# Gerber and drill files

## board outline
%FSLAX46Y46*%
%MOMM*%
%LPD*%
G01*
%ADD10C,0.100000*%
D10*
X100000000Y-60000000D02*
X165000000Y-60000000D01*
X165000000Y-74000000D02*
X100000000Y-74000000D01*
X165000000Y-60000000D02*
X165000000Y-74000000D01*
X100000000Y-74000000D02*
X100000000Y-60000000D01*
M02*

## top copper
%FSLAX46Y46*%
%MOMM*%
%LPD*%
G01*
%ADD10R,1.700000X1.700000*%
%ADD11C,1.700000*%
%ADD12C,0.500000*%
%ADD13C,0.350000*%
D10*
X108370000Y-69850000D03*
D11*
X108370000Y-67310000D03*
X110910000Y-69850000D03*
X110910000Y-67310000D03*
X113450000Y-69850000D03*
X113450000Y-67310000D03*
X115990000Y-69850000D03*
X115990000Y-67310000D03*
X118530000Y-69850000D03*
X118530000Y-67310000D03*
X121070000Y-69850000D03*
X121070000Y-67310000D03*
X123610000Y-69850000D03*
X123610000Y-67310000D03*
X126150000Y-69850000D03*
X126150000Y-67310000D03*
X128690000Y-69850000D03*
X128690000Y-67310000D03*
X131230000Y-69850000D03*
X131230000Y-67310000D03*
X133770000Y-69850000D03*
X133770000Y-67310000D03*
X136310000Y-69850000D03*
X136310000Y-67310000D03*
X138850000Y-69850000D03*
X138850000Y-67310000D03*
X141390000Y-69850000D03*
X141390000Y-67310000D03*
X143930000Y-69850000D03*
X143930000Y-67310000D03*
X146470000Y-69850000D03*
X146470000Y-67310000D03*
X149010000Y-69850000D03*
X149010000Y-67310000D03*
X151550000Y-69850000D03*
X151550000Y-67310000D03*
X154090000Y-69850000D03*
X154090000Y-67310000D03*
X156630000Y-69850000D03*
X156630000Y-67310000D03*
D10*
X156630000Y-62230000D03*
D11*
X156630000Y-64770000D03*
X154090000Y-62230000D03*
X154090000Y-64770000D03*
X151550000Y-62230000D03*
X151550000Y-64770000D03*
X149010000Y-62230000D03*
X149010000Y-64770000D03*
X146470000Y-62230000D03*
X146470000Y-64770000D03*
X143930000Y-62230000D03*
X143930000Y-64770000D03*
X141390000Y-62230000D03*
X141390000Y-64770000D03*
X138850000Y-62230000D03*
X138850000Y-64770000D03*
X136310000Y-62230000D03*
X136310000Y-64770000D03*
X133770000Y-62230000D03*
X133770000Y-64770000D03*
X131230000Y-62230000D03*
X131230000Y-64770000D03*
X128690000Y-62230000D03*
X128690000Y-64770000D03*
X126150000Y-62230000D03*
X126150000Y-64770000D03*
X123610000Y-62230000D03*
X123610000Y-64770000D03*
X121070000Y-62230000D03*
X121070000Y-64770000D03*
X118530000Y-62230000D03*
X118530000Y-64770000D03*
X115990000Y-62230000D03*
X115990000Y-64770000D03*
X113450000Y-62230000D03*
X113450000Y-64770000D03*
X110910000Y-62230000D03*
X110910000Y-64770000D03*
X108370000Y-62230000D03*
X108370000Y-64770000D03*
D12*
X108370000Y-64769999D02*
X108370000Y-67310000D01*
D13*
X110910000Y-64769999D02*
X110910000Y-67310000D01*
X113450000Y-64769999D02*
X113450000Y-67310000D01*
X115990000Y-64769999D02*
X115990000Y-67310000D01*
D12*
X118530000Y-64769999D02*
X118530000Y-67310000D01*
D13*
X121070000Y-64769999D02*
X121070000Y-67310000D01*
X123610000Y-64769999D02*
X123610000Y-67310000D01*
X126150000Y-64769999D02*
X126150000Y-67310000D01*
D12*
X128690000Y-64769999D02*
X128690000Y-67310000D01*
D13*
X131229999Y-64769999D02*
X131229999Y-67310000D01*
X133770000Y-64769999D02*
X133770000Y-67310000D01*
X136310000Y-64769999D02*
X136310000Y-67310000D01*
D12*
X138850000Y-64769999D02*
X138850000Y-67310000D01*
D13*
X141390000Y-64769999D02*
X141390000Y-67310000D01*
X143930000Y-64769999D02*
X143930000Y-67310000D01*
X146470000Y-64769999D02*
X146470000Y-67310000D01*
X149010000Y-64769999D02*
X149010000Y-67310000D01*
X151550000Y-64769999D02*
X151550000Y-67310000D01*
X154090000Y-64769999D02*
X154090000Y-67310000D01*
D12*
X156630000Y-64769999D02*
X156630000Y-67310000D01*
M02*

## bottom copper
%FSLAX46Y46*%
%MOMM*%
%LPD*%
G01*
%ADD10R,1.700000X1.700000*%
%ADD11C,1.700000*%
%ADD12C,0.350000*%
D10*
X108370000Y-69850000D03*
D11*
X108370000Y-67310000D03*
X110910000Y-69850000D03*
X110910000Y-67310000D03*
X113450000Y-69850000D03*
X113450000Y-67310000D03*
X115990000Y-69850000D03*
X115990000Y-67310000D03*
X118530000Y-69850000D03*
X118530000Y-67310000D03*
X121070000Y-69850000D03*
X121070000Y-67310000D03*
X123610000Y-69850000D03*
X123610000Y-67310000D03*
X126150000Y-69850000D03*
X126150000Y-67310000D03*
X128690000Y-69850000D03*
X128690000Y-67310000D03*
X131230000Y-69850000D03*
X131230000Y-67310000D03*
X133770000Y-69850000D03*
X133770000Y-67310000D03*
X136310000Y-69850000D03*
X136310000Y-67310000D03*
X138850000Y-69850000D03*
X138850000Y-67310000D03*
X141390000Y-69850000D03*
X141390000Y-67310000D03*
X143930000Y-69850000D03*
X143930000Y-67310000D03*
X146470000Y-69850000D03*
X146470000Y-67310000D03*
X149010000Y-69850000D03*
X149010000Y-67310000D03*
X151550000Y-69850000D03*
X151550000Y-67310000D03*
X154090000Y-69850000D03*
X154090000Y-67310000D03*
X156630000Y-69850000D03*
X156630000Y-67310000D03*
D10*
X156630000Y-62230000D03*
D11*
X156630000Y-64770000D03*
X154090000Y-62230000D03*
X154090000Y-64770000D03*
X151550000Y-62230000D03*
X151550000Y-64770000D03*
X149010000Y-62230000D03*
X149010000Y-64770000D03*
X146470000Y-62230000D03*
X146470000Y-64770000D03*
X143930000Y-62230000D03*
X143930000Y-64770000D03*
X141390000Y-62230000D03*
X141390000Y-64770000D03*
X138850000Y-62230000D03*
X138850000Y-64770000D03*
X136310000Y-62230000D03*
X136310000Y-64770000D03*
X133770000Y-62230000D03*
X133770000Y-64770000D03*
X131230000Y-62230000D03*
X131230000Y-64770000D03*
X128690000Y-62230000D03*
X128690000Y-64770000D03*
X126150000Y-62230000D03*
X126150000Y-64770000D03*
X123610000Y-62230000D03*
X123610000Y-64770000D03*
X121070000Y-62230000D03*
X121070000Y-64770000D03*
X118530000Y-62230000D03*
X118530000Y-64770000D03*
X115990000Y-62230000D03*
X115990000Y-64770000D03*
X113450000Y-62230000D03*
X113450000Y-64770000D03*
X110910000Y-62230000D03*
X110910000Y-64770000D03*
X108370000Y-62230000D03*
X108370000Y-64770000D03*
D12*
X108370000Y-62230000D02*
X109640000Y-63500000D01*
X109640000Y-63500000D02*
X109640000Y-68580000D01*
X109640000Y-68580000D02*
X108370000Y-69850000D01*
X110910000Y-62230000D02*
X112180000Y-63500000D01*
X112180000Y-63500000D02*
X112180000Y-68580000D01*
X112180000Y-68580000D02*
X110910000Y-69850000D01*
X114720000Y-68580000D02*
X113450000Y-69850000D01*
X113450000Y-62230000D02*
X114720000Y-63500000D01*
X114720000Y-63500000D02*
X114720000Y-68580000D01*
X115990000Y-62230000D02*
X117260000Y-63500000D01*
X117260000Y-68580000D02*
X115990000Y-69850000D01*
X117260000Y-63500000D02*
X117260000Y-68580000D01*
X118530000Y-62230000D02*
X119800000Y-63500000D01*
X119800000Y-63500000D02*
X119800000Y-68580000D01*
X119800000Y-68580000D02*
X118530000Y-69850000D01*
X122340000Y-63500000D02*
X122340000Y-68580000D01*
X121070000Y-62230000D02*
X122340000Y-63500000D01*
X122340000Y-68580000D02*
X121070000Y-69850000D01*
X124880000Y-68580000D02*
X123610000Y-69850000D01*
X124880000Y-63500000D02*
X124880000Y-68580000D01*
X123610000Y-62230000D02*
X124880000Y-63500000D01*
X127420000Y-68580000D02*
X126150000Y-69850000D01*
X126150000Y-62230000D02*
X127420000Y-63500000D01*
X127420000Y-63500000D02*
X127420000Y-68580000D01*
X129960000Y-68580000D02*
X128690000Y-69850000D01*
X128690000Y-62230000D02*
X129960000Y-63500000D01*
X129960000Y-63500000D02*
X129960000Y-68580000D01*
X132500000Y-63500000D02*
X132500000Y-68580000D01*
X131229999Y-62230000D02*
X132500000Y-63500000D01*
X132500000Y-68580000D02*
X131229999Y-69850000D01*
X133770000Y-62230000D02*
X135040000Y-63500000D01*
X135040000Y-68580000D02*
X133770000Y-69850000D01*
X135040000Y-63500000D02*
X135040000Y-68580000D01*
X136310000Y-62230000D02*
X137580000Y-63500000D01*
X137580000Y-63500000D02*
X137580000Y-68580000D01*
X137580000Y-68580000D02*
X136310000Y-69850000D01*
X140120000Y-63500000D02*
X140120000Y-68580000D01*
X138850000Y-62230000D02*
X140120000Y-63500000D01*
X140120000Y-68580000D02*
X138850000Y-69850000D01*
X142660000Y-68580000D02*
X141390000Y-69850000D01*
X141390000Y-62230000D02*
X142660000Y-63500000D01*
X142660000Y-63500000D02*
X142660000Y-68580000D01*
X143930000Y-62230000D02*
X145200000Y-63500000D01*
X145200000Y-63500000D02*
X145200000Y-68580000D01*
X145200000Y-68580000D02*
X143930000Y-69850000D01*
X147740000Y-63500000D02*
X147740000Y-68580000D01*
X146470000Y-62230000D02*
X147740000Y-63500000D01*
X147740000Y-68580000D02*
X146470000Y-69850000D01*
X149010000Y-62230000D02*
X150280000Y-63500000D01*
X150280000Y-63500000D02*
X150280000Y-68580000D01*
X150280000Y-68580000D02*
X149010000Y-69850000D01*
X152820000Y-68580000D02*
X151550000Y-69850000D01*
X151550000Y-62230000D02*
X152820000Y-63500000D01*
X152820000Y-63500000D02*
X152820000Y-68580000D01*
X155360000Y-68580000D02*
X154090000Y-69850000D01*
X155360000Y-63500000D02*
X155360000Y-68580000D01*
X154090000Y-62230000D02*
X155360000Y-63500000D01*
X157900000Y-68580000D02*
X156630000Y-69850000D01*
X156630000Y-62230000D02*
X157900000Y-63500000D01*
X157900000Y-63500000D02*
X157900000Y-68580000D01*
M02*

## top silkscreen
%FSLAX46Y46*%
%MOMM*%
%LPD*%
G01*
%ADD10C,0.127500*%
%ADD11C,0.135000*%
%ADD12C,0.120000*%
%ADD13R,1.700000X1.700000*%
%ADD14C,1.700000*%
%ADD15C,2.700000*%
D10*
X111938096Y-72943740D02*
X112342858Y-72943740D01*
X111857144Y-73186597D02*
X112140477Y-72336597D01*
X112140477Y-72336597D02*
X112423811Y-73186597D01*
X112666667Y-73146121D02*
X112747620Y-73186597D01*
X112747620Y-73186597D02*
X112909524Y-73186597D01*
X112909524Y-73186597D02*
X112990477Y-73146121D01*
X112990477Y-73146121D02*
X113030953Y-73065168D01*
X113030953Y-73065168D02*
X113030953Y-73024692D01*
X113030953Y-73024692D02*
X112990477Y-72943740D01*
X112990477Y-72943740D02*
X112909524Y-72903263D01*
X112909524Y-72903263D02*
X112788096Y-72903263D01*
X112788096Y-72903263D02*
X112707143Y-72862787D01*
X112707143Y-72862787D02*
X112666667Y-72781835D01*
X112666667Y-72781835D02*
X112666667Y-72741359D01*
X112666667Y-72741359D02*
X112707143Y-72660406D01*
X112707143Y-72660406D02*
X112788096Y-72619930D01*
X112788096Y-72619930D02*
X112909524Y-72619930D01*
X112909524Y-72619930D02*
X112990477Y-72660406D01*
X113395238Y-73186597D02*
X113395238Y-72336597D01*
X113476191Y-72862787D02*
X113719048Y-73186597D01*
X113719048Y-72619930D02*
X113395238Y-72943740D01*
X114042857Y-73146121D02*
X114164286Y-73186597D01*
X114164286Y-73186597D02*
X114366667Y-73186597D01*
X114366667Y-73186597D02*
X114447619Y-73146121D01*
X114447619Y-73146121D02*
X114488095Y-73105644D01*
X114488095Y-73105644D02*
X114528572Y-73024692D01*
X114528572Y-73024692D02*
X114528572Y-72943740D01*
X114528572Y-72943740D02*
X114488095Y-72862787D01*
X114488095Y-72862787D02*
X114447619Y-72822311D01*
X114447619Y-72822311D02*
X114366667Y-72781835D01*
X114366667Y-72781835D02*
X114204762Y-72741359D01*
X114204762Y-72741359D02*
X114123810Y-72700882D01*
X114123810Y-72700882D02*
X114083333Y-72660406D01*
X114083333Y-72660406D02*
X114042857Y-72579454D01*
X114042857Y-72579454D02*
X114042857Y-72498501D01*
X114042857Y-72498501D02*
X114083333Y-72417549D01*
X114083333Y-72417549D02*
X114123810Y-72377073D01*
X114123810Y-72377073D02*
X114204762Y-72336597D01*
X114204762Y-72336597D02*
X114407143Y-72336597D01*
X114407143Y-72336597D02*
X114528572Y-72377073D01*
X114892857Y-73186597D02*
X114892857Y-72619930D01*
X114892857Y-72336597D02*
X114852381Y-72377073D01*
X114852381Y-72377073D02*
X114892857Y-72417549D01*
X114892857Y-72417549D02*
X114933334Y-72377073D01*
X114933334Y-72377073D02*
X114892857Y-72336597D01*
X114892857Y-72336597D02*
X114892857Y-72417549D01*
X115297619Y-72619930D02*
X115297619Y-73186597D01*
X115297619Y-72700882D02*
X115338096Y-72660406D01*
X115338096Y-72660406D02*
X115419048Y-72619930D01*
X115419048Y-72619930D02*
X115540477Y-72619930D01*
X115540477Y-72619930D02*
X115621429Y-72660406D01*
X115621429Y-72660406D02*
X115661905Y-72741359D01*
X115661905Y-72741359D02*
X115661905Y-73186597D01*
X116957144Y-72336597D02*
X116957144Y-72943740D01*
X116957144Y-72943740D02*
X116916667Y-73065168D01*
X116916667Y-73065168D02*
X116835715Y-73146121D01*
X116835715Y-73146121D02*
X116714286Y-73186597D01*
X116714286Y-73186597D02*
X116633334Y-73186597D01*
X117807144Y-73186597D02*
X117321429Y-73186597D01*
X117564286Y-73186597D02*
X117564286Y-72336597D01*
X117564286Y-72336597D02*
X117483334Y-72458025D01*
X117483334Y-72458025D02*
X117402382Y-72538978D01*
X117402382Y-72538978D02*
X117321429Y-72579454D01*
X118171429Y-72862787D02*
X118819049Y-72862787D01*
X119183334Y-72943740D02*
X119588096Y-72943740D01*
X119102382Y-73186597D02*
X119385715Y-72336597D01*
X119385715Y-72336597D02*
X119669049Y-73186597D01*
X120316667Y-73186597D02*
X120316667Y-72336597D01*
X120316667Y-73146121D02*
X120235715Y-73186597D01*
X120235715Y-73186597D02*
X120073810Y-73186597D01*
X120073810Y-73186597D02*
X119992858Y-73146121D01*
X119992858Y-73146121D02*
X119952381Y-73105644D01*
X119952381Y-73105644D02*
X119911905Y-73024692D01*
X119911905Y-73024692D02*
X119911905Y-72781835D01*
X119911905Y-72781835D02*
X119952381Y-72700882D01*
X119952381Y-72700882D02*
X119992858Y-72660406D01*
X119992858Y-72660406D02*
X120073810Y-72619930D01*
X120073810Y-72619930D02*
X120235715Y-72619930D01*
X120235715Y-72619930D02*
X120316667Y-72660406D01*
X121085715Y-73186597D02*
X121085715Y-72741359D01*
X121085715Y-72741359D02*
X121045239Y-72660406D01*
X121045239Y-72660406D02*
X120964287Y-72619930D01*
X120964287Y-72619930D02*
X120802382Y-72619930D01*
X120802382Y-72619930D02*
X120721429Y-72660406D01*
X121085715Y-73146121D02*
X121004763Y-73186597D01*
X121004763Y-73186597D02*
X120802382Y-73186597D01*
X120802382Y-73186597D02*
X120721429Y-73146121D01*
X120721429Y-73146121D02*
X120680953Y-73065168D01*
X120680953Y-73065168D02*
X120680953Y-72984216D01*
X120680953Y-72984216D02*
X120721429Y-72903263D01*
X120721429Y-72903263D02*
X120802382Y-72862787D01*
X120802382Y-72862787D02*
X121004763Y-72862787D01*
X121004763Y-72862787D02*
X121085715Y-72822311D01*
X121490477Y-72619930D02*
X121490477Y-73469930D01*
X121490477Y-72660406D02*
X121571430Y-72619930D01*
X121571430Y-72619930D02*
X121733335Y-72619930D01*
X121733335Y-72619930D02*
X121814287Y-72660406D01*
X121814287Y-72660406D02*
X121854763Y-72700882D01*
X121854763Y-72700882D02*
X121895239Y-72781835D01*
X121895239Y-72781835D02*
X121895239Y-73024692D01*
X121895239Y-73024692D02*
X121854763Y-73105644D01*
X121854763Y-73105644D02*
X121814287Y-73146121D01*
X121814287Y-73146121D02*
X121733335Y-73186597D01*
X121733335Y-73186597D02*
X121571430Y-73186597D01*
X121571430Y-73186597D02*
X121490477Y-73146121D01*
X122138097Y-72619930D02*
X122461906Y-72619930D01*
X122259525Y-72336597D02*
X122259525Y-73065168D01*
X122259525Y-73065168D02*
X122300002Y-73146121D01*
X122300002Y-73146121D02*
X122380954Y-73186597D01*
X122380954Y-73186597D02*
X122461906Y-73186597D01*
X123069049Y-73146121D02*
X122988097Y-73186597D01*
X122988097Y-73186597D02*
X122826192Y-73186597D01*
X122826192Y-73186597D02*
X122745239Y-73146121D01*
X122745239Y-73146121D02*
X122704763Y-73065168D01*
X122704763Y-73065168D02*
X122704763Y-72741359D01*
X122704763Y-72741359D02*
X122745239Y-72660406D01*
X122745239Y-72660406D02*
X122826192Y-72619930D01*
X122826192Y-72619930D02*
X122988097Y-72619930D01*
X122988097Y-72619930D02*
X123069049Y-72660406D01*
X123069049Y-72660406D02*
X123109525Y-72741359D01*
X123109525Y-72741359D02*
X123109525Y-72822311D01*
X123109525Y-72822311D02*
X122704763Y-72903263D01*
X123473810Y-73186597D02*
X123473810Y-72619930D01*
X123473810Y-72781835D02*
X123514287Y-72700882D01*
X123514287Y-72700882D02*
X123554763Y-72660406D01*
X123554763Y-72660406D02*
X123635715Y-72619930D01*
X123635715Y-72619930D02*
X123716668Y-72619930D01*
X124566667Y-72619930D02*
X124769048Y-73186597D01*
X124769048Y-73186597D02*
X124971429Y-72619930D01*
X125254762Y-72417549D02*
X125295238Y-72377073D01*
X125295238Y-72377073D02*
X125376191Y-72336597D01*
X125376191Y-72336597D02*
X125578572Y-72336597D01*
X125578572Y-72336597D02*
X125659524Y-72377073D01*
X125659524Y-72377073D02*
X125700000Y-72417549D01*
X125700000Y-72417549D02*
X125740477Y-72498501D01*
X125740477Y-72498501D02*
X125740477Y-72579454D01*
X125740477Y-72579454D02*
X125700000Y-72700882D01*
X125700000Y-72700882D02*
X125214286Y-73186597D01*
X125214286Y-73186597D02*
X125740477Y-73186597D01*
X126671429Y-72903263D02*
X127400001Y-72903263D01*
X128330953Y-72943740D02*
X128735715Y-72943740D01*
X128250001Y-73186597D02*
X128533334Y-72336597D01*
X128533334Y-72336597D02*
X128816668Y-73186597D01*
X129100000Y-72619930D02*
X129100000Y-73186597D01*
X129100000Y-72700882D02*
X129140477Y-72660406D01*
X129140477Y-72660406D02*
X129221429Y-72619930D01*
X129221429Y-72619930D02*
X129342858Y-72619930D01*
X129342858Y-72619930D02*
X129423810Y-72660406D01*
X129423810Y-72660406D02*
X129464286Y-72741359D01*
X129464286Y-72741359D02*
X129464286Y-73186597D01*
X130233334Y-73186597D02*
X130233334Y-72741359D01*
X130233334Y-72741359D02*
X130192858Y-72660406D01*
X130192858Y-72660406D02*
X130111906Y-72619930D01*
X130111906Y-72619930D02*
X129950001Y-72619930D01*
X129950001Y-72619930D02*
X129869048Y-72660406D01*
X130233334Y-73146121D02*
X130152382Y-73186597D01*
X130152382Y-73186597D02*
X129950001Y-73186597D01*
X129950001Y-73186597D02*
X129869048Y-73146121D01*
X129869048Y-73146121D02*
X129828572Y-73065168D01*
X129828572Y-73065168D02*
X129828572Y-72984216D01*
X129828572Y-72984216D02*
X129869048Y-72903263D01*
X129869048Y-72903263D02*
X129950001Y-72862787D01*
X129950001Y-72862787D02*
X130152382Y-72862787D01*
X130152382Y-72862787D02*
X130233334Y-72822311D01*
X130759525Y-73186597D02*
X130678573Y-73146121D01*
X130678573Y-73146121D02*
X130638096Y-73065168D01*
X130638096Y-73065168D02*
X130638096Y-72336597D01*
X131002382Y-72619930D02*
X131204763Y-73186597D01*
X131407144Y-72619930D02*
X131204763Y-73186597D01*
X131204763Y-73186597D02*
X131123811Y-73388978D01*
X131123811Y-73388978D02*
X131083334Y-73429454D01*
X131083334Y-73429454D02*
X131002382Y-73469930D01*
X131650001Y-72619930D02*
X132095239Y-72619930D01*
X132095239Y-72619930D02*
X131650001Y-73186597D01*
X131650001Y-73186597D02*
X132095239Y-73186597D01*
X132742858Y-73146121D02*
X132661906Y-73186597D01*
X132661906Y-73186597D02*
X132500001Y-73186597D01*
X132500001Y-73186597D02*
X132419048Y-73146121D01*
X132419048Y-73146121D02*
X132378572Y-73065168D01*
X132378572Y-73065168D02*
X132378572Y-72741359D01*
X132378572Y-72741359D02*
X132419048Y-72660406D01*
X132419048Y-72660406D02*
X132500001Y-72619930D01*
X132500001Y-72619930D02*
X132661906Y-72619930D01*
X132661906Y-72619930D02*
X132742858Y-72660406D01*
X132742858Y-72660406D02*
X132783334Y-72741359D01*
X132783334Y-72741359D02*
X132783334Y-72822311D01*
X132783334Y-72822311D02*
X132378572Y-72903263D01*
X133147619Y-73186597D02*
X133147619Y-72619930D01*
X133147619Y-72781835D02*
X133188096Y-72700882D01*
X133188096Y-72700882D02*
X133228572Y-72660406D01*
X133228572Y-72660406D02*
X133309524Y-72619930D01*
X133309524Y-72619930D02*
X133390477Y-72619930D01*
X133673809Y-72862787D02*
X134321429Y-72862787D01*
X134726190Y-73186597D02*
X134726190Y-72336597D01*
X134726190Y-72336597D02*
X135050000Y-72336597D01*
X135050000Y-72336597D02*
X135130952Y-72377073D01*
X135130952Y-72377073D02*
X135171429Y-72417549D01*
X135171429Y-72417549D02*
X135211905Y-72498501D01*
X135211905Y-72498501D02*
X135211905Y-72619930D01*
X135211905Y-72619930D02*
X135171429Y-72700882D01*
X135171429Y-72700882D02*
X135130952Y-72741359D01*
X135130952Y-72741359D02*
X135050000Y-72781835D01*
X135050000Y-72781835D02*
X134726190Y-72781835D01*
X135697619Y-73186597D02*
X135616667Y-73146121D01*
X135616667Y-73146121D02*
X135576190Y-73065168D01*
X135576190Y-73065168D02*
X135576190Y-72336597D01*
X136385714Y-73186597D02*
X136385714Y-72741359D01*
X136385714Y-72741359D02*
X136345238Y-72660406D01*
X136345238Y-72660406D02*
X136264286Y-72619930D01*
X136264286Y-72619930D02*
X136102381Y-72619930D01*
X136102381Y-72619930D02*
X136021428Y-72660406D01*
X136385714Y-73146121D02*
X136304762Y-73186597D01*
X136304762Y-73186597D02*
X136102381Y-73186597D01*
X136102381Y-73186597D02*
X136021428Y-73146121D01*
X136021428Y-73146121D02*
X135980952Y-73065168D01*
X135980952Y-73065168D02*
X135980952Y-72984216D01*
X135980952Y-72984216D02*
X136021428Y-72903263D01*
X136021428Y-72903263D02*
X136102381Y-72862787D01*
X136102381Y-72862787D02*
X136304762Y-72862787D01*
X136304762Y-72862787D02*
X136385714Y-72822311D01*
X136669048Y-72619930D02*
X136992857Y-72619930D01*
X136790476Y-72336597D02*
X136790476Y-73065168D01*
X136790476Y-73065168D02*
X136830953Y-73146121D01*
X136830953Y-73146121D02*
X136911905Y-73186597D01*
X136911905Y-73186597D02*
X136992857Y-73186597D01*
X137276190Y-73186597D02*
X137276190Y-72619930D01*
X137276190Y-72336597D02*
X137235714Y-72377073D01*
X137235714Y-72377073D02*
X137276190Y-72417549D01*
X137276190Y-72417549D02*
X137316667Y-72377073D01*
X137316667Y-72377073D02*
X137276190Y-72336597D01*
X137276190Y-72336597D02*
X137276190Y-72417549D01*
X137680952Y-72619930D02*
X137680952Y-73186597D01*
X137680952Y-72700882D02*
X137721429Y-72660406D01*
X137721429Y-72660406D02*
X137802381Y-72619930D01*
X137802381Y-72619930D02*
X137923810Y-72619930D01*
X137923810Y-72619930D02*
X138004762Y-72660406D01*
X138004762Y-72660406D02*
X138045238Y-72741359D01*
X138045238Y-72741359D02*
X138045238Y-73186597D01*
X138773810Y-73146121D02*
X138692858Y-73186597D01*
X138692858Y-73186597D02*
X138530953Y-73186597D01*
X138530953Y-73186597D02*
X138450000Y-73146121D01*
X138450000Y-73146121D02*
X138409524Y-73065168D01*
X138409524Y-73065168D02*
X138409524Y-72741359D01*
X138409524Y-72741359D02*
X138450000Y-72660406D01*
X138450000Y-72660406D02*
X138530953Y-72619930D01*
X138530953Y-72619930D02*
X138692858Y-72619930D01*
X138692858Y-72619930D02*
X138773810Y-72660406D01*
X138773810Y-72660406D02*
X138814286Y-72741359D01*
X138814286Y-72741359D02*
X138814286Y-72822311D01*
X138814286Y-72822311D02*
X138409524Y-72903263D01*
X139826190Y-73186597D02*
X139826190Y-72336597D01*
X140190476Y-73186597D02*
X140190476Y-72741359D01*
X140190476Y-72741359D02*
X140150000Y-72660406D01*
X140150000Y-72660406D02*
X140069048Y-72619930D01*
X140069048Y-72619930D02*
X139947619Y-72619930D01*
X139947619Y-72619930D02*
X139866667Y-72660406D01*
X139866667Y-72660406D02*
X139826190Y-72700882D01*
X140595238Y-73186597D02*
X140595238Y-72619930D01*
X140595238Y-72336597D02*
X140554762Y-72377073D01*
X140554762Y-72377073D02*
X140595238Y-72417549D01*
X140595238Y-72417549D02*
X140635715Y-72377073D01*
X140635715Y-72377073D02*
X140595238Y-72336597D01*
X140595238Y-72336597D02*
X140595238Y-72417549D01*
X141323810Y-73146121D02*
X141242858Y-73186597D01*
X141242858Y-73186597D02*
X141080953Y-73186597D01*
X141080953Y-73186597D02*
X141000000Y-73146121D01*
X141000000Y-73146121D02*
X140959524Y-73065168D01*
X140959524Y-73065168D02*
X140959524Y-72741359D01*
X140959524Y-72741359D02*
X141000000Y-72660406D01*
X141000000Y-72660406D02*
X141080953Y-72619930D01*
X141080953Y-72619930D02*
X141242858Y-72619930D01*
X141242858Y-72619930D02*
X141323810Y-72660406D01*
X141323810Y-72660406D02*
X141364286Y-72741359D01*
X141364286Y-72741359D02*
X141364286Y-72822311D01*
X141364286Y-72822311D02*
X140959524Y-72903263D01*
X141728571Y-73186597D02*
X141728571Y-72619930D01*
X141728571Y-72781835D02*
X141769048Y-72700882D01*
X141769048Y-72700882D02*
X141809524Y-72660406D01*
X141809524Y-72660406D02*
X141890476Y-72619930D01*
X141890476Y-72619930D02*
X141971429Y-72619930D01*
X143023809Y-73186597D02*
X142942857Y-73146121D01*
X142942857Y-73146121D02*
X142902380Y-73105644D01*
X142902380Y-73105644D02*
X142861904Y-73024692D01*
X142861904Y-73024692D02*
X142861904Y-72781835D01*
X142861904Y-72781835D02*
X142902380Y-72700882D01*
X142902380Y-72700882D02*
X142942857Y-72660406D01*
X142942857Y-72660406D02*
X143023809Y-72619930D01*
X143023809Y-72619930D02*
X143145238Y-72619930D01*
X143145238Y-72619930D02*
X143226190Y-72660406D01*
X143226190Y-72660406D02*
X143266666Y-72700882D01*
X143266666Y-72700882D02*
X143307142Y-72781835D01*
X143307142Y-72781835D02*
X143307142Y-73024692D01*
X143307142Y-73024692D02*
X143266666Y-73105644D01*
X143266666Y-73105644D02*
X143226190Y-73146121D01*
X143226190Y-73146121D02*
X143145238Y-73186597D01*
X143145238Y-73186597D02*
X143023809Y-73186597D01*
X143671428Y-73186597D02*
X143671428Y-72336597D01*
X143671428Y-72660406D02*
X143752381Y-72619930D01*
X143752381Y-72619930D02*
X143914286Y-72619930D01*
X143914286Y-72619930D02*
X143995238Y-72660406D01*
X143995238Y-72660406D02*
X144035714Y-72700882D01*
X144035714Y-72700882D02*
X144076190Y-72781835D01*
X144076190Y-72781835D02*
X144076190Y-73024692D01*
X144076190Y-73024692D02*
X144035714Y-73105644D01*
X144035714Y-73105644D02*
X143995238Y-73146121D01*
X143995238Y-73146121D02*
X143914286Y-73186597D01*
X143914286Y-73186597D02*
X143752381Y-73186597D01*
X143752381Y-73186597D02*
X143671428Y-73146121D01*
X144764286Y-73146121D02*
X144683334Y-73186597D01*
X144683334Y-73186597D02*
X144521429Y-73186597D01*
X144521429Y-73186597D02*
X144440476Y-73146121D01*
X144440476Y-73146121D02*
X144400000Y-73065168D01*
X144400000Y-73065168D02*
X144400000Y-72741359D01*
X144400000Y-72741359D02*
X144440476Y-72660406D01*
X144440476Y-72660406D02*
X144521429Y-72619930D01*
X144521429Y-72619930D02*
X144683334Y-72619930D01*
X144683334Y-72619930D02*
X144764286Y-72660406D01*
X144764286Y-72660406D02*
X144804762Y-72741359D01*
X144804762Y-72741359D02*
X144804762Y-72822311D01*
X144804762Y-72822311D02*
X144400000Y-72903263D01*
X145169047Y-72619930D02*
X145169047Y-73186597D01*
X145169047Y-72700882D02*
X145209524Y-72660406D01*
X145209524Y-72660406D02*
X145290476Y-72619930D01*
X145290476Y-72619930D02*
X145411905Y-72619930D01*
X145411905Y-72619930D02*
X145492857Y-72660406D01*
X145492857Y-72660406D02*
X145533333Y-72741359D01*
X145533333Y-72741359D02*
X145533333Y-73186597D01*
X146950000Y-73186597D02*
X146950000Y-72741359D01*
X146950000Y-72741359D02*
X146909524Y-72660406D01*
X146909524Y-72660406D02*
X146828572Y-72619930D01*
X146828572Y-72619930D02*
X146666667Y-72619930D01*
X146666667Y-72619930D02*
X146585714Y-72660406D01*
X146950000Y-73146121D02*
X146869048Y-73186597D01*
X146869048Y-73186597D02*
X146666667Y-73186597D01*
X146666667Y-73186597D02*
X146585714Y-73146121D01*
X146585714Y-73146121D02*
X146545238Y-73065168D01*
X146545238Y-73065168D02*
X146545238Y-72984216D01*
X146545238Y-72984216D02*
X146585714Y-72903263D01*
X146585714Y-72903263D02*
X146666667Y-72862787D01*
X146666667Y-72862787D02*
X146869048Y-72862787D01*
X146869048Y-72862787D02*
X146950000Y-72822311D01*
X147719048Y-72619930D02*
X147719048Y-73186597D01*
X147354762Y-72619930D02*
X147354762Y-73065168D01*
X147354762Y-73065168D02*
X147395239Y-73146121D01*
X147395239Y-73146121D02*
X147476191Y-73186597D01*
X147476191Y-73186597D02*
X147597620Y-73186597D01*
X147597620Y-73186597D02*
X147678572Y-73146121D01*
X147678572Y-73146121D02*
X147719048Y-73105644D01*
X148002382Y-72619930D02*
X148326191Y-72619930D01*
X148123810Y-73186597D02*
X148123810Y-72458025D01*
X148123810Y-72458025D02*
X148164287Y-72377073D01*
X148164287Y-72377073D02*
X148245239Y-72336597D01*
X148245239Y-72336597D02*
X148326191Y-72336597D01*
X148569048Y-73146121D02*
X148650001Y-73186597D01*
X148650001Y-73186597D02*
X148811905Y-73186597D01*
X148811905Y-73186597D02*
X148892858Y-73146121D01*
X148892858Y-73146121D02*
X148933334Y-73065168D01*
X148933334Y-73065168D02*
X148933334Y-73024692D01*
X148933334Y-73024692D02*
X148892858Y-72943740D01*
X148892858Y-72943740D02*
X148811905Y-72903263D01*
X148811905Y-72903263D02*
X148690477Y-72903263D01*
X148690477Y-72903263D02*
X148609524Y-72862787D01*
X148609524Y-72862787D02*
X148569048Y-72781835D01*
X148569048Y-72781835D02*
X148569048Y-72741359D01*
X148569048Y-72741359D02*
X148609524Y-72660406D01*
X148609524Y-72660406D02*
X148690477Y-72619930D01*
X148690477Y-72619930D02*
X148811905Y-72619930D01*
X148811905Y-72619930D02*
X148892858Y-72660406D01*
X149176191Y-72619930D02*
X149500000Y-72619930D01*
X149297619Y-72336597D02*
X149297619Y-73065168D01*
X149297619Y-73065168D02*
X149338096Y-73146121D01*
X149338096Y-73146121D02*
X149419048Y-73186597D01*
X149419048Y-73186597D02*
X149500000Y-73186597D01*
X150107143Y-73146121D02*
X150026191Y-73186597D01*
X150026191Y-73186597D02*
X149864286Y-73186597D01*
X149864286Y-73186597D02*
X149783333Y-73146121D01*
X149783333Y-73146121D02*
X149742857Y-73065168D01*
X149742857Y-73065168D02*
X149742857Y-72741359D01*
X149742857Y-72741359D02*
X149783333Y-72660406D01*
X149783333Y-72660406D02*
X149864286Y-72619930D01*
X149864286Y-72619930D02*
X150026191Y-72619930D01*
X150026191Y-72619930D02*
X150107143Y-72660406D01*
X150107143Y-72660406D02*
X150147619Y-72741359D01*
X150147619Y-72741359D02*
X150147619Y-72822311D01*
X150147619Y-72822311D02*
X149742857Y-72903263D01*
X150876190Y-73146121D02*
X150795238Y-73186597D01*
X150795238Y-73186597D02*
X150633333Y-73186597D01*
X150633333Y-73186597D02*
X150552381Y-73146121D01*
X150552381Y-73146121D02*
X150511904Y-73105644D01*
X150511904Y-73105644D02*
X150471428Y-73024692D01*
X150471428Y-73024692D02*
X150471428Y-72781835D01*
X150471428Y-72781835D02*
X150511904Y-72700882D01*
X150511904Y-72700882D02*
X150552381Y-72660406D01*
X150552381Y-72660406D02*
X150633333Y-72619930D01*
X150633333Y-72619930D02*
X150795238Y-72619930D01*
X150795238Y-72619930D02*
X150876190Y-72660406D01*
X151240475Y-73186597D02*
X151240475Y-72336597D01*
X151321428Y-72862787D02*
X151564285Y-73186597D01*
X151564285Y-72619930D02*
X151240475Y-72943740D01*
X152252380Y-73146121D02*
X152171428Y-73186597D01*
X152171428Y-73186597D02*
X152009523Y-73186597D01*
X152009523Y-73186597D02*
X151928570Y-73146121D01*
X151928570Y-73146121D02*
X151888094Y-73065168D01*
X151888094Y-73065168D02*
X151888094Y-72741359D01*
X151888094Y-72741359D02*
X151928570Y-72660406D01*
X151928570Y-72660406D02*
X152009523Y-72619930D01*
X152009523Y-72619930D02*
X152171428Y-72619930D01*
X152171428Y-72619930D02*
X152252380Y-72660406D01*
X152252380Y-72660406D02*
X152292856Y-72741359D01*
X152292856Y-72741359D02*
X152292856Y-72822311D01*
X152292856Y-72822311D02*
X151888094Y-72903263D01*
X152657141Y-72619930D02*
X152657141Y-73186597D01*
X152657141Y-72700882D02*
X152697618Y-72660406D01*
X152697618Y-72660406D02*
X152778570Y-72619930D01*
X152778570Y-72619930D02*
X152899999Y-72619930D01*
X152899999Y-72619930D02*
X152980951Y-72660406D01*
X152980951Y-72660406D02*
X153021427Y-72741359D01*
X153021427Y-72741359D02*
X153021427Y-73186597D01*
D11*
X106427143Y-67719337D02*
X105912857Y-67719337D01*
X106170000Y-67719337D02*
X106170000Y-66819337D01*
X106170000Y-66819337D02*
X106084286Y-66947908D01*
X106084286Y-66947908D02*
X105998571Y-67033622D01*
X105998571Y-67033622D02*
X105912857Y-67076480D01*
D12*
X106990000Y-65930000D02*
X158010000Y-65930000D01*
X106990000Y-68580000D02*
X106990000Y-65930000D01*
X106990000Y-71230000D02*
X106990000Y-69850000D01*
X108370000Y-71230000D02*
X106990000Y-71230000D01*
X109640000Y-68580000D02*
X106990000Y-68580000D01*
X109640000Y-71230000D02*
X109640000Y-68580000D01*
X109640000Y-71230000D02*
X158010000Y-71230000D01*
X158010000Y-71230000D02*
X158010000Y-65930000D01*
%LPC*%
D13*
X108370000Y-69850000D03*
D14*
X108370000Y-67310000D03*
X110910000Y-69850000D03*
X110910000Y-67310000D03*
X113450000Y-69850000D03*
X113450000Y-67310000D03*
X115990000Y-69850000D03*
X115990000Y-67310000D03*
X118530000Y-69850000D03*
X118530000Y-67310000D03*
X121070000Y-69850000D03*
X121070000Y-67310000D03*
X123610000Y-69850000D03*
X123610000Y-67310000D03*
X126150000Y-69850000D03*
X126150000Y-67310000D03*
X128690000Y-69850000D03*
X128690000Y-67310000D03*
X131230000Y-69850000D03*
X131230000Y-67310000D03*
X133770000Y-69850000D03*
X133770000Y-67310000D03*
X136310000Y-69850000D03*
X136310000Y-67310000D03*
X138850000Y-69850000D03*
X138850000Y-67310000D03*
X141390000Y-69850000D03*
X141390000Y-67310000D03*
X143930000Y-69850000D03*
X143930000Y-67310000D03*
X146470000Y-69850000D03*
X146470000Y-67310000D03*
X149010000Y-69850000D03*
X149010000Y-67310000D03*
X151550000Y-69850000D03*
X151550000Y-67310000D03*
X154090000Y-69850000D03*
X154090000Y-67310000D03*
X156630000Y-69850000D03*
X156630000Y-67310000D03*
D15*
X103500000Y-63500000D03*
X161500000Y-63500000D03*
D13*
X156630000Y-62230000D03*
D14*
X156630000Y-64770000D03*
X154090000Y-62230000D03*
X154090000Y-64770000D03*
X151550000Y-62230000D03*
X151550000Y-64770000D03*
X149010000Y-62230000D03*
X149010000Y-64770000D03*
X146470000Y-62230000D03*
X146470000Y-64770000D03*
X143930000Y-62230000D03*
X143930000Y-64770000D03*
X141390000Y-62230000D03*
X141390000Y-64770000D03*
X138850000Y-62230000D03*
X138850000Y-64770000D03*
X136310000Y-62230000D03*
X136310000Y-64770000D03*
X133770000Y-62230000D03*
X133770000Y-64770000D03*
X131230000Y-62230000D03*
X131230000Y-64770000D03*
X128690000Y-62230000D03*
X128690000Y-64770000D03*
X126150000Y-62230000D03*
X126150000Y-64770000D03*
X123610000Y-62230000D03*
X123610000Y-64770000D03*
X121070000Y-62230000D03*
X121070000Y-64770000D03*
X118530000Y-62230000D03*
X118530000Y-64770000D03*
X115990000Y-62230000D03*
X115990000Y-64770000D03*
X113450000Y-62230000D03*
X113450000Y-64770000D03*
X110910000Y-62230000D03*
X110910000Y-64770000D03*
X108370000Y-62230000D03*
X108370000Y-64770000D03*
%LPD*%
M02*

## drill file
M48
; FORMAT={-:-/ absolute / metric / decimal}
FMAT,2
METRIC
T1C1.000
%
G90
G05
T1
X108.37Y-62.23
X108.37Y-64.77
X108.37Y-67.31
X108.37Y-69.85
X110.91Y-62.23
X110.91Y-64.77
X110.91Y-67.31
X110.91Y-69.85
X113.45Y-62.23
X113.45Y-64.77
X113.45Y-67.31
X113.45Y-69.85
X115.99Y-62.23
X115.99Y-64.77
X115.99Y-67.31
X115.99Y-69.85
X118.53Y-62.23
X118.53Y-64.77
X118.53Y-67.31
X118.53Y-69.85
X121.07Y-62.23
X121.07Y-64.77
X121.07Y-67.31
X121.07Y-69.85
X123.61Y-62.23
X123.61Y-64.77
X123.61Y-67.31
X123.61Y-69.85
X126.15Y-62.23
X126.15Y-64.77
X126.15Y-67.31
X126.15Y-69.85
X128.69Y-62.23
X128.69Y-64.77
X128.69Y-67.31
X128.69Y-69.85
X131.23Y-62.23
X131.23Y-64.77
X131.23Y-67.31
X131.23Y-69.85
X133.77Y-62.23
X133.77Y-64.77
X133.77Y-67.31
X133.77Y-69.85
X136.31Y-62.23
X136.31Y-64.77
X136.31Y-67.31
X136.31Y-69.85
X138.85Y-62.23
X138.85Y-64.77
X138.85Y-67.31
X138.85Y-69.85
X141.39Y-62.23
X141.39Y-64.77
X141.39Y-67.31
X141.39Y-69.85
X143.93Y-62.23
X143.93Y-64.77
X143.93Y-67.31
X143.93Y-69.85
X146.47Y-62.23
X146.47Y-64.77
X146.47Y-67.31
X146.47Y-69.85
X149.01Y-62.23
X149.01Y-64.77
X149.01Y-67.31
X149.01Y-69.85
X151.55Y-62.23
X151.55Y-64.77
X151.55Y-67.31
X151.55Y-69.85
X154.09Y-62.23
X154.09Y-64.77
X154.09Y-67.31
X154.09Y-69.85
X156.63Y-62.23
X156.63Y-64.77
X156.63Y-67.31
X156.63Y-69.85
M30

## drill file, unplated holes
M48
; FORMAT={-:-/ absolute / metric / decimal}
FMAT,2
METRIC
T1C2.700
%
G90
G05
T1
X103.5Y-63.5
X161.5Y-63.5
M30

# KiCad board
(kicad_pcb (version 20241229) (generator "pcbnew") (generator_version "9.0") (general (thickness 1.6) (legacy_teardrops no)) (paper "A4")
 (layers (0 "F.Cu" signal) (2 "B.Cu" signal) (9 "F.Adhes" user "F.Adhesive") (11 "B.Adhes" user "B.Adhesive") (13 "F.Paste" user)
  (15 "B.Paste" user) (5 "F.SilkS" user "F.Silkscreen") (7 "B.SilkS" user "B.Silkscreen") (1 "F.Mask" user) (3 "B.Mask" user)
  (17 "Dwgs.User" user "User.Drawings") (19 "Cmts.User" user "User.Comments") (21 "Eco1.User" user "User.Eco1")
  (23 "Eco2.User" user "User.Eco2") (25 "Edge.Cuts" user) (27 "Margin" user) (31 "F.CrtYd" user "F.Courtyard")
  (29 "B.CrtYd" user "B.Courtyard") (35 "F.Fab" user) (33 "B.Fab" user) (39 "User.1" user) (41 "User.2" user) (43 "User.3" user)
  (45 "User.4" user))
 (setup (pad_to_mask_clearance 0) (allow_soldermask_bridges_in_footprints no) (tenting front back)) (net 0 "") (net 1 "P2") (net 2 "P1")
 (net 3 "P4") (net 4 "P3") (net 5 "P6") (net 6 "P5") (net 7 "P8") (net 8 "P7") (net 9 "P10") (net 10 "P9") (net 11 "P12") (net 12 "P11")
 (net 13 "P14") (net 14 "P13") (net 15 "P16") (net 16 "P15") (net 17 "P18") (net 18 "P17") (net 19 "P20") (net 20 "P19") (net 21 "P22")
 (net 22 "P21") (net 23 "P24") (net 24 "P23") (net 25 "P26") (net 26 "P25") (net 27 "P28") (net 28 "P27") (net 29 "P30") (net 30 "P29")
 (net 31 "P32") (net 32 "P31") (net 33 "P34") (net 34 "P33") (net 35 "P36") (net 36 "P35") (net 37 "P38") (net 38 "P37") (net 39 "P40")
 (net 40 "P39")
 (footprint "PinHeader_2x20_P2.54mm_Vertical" (layer "F.Cu") (at 108.37 69.85 90)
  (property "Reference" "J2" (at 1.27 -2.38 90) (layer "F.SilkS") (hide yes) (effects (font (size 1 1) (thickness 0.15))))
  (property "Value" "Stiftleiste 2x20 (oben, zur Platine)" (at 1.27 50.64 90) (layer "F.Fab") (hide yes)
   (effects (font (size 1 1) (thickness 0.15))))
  (fp_line (start 3.92 -1.38) (end 3.92 49.64) (stroke (width 0.12) (type solid)) (layer "F.SilkS"))
  (fp_line (start 1.27 -1.38) (end 3.92 -1.38) (stroke (width 0.12) (type solid)) (layer "F.SilkS"))
  (fp_line (start -1.38 -1.38) (end 0 -1.38) (stroke (width 0.12) (type solid)) (layer "F.SilkS"))
  (fp_line (start -1.38 0) (end -1.38 -1.38) (stroke (width 0.12) (type solid)) (layer "F.SilkS"))
  (fp_line (start 1.27 1.27) (end 1.27 -1.38) (stroke (width 0.12) (type solid)) (layer "F.SilkS"))
  (fp_line (start -1.38 1.27) (end 1.27 1.27) (stroke (width 0.12) (type solid)) (layer "F.SilkS"))
  (fp_line (start -1.38 1.27) (end -1.38 49.64) (stroke (width 0.12) (type solid)) (layer "F.SilkS"))
  (fp_line (start -1.38 49.64) (end 3.92 49.64) (stroke (width 0.12) (type solid)) (layer "F.SilkS"))
  (pad "1" thru_hole rect (at 0 0 90) (size 1.7 1.7) (drill 1) (layers "*.Cu" "*.Mask") (remove_unused_layers no) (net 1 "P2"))
  (pad "2" thru_hole circle (at 2.54 0 90) (size 1.7 1.7) (drill 1) (layers "*.Cu" "*.Mask") (remove_unused_layers no) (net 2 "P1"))
  (pad "3" thru_hole circle (at 0 2.54 90) (size 1.7 1.7) (drill 1) (layers "*.Cu" "*.Mask") (remove_unused_layers no) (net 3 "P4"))
  (pad "4" thru_hole circle (at 2.54 2.54 90) (size 1.7 1.7) (drill 1) (layers "*.Cu" "*.Mask") (remove_unused_layers no) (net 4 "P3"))
  (pad "5" thru_hole circle (at 0 5.08 90) (size 1.7 1.7) (drill 1) (layers "*.Cu" "*.Mask") (remove_unused_layers no) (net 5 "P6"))
  (pad "6" thru_hole circle (at 2.54 5.08 90) (size 1.7 1.7) (drill 1) (layers "*.Cu" "*.Mask") (remove_unused_layers no) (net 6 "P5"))
  (pad "7" thru_hole circle (at 0 7.62 90) (size 1.7 1.7) (drill 1) (layers "*.Cu" "*.Mask") (remove_unused_layers no) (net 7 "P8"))
  (pad "8" thru_hole circle (at 2.54 7.62 90) (size 1.7 1.7) (drill 1) (layers "*.Cu" "*.Mask") (remove_unused_layers no) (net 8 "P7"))
  (pad "9" thru_hole circle (at 0 10.16 90) (size 1.7 1.7) (drill 1) (layers "*.Cu" "*.Mask") (remove_unused_layers no) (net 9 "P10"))
  (pad "10" thru_hole circle (at 2.54 10.16 90) (size 1.7 1.7) (drill 1) (layers "*.Cu" "*.Mask") (remove_unused_layers no) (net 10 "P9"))
  (pad "11" thru_hole circle (at 0 12.7 90) (size 1.7 1.7) (drill 1) (layers "*.Cu" "*.Mask") (remove_unused_layers no) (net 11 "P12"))
  (pad "12" thru_hole circle (at 2.54 12.7 90) (size 1.7 1.7) (drill 1) (layers "*.Cu" "*.Mask") (remove_unused_layers no) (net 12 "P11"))
  (pad "13" thru_hole circle (at 0 15.24 90) (size 1.7 1.7) (drill 1) (layers "*.Cu" "*.Mask") (remove_unused_layers no) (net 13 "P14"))
  (pad "14" thru_hole circle (at 2.54 15.24 90) (size 1.7 1.7) (drill 1) (layers "*.Cu" "*.Mask") (remove_unused_layers no) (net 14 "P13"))
  (pad "15" thru_hole circle (at 0 17.78 90) (size 1.7 1.7) (drill 1) (layers "*.Cu" "*.Mask") (remove_unused_layers no) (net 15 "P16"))
  (pad "16" thru_hole circle (at 2.54 17.78 90) (size 1.7 1.7) (drill 1) (layers "*.Cu" "*.Mask") (remove_unused_layers no) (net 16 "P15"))
  (pad "17" thru_hole circle (at 0 20.32 90) (size 1.7 1.7) (drill 1) (layers "*.Cu" "*.Mask") (remove_unused_layers no) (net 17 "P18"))
  (pad "18" thru_hole circle (at 2.54 20.32 90) (size 1.7 1.7) (drill 1) (layers "*.Cu" "*.Mask") (remove_unused_layers no) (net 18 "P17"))
  (pad "19" thru_hole circle (at 0 22.86 90) (size 1.7 1.7) (drill 1) (layers "*.Cu" "*.Mask") (remove_unused_layers no) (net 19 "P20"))
  (pad "20" thru_hole circle (at 2.54 22.86 90) (size 1.7 1.7) (drill 1) (layers "*.Cu" "*.Mask") (remove_unused_layers no) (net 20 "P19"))
  (pad "21" thru_hole circle (at 0 25.4 90) (size 1.7 1.7) (drill 1) (layers "*.Cu" "*.Mask") (remove_unused_layers no) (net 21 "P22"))
  (pad "22" thru_hole circle (at 2.54 25.4 90) (size 1.7 1.7) (drill 1) (layers "*.Cu" "*.Mask") (remove_unused_layers no) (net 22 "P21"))
  (pad "23" thru_hole circle (at 0 27.94 90) (size 1.7 1.7) (drill 1) (layers "*.Cu" "*.Mask") (remove_unused_layers no) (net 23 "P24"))
  (pad "24" thru_hole circle (at 2.54 27.94 90) (size 1.7 1.7) (drill 1) (layers "*.Cu" "*.Mask") (remove_unused_layers no) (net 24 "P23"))
  (pad "25" thru_hole circle (at 0 30.48 90) (size 1.7 1.7) (drill 1) (layers "*.Cu" "*.Mask") (remove_unused_layers no) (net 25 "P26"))
  (pad "26" thru_hole circle (at 2.54 30.48 90) (size 1.7 1.7) (drill 1) (layers "*.Cu" "*.Mask") (remove_unused_layers no) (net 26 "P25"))
  (pad "27" thru_hole circle (at 0 33.02 90) (size 1.7 1.7) (drill 1) (layers "*.Cu" "*.Mask") (remove_unused_layers no) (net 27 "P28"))
  (pad "28" thru_hole circle (at 2.54 33.02 90) (size 1.7 1.7) (drill 1) (layers "*.Cu" "*.Mask") (remove_unused_layers no) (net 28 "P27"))
  (pad "29" thru_hole circle (at 0 35.56 90) (size 1.7 1.7) (drill 1) (layers "*.Cu" "*.Mask") (remove_unused_layers no) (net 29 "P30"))
  (pad "30" thru_hole circle (at 2.54 35.56 90) (size 1.7 1.7) (drill 1) (layers "*.Cu" "*.Mask") (remove_unused_layers no) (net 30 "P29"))
  (pad "31" thru_hole circle (at 0 38.1 90) (size 1.7 1.7) (drill 1) (layers "*.Cu" "*.Mask") (remove_unused_layers no) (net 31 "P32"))
  (pad "32" thru_hole circle (at 2.54 38.1 90) (size 1.7 1.7) (drill 1) (layers "*.Cu" "*.Mask") (remove_unused_layers no) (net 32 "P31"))
  (pad "33" thru_hole circle (at 0 40.64 90) (size 1.7 1.7) (drill 1) (layers "*.Cu" "*.Mask") (remove_unused_layers no) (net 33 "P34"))
  (pad "34" thru_hole circle (at 2.54 40.64 90) (size 1.7 1.7) (drill 1) (layers "*.Cu" "*.Mask") (remove_unused_layers no) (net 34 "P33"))
  (pad "35" thru_hole circle (at 0 43.18 90) (size 1.7 1.7) (drill 1) (layers "*.Cu" "*.Mask") (remove_unused_layers no) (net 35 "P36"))
  (pad "36" thru_hole circle (at 2.54 43.18 90) (size 1.7 1.7) (drill 1) (layers "*.Cu" "*.Mask") (remove_unused_layers no) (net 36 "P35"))
  (pad "37" thru_hole circle (at 0 45.72 90) (size 1.7 1.7) (drill 1) (layers "*.Cu" "*.Mask") (remove_unused_layers no) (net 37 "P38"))
  (pad "38" thru_hole circle (at 2.54 45.72 90) (size 1.7 1.7) (drill 1) (layers "*.Cu" "*.Mask") (remove_unused_layers no) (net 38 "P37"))
  (pad "39" thru_hole circle (at 0 48.26 90) (size 1.7 1.7) (drill 1) (layers "*.Cu" "*.Mask") (remove_unused_layers no) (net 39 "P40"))
  (pad "40" thru_hole circle (at 2.54 48.26 90) (size 1.7 1.7) (drill 1) (layers "*.Cu" "*.Mask") (remove_unused_layers no) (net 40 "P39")))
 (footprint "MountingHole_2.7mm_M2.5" (layer "F.Cu") (at 103.5 63.5)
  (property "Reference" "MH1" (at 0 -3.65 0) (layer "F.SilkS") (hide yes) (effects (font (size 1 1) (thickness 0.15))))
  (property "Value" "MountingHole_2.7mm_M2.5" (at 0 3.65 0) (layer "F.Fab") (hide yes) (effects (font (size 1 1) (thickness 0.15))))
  (pad "" np_thru_hole circle (at 0 0) (size 2.7 2.7) (drill 2.7) (layers "*.Cu" "*.Mask")))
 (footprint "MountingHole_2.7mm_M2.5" (layer "F.Cu") (at 161.5 63.5)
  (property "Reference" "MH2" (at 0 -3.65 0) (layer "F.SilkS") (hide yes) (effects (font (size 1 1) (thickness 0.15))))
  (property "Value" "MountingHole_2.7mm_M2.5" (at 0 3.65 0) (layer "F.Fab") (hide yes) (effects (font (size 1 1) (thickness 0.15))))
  (pad "" np_thru_hole circle (at 0 0) (size 2.7 2.7) (drill 2.7) (layers "*.Cu" "*.Mask")))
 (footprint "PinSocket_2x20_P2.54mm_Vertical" (layer "B.Cu") (at 156.63 62.23 90)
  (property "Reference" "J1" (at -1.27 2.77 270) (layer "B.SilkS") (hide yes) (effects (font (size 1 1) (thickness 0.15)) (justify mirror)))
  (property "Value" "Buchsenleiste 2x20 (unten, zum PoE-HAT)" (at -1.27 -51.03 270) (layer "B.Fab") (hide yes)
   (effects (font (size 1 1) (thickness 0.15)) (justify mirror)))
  (pad "1" thru_hole rect (at 0 0 90) (size 1.7 1.7) (drill 1) (layers "*.Cu" "*.Mask") (remove_unused_layers no) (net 39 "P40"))
  (pad "2" thru_hole circle (at -2.54 0 90) (size 1.7 1.7) (drill 1) (layers "*.Cu" "*.Mask") (remove_unused_layers no) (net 40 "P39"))
  (pad "3" thru_hole circle (at 0 -2.54 90) (size 1.7 1.7) (drill 1) (layers "*.Cu" "*.Mask") (remove_unused_layers no) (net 37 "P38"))
  (pad "4" thru_hole circle (at -2.54 -2.54 90) (size 1.7 1.7) (drill 1) (layers "*.Cu" "*.Mask") (remove_unused_layers no) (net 38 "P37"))
  (pad "5" thru_hole circle (at 0 -5.08 90) (size 1.7 1.7) (drill 1) (layers "*.Cu" "*.Mask") (remove_unused_layers no) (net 35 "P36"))
  (pad "6" thru_hole circle (at -2.54 -5.08 90) (size 1.7 1.7) (drill 1) (layers "*.Cu" "*.Mask") (remove_unused_layers no) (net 36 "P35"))
  (pad "7" thru_hole circle (at 0 -7.62 90) (size 1.7 1.7) (drill 1) (layers "*.Cu" "*.Mask") (remove_unused_layers no) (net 33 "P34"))
  (pad "8" thru_hole circle (at -2.54 -7.62 90) (size 1.7 1.7) (drill 1) (layers "*.Cu" "*.Mask") (remove_unused_layers no) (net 34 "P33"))
  (pad "9" thru_hole circle (at 0 -10.16 90) (size 1.7 1.7) (drill 1) (layers "*.Cu" "*.Mask") (remove_unused_layers no) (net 31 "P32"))
  (pad "10" thru_hole circle (at -2.54 -10.16 90) (size 1.7 1.7) (drill 1) (layers "*.Cu" "*.Mask") (remove_unused_layers no) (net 32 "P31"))
  (pad "11" thru_hole circle (at 0 -12.7 90) (size 1.7 1.7) (drill 1) (layers "*.Cu" "*.Mask") (remove_unused_layers no) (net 29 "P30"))
  (pad "12" thru_hole circle (at -2.54 -12.7 90) (size 1.7 1.7) (drill 1) (layers "*.Cu" "*.Mask") (remove_unused_layers no) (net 30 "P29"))
  (pad "13" thru_hole circle (at 0 -15.24 90) (size 1.7 1.7) (drill 1) (layers "*.Cu" "*.Mask") (remove_unused_layers no) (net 27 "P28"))
  (pad "14" thru_hole circle (at -2.54 -15.24 90) (size 1.7 1.7) (drill 1) (layers "*.Cu" "*.Mask") (remove_unused_layers no) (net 28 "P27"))
  (pad "15" thru_hole circle (at 0 -17.78 90) (size 1.7 1.7) (drill 1) (layers "*.Cu" "*.Mask") (remove_unused_layers no) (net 25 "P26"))
  (pad "16" thru_hole circle (at -2.54 -17.78 90) (size 1.7 1.7) (drill 1) (layers "*.Cu" "*.Mask") (remove_unused_layers no) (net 26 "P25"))
  (pad "17" thru_hole circle (at 0 -20.32 90) (size 1.7 1.7) (drill 1) (layers "*.Cu" "*.Mask") (remove_unused_layers no) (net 23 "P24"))
  (pad "18" thru_hole circle (at -2.54 -20.32 90) (size 1.7 1.7) (drill 1) (layers "*.Cu" "*.Mask") (remove_unused_layers no) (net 24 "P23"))
  (pad "19" thru_hole circle (at 0 -22.86 90) (size 1.7 1.7) (drill 1) (layers "*.Cu" "*.Mask") (remove_unused_layers no) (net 21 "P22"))
  (pad "20" thru_hole circle (at -2.54 -22.86 90) (size 1.7 1.7) (drill 1) (layers "*.Cu" "*.Mask") (remove_unused_layers no) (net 22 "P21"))
  (pad "21" thru_hole circle (at 0 -25.4 90) (size 1.7 1.7) (drill 1) (layers "*.Cu" "*.Mask") (remove_unused_layers no) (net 19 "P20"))
  (pad "22" thru_hole circle (at -2.54 -25.4 90) (size 1.7 1.7) (drill 1) (layers "*.Cu" "*.Mask") (remove_unused_layers no) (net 20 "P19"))
  (pad "23" thru_hole circle (at 0 -27.94 90) (size 1.7 1.7) (drill 1) (layers "*.Cu" "*.Mask") (remove_unused_layers no) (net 17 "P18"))
  (pad "24" thru_hole circle (at -2.54 -27.94 90) (size 1.7 1.7) (drill 1) (layers "*.Cu" "*.Mask") (remove_unused_layers no) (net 18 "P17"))
  (pad "25" thru_hole circle (at 0 -30.48 90) (size 1.7 1.7) (drill 1) (layers "*.Cu" "*.Mask") (remove_unused_layers no) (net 15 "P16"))
  (pad "26" thru_hole circle (at -2.54 -30.48 90) (size 1.7 1.7) (drill 1) (layers "*.Cu" "*.Mask") (remove_unused_layers no) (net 16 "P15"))
  (pad "27" thru_hole circle (at 0 -33.02 90) (size 1.7 1.7) (drill 1) (layers "*.Cu" "*.Mask") (remove_unused_layers no) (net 13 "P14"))
  (pad "28" thru_hole circle (at -2.54 -33.02 90) (size 1.7 1.7) (drill 1) (layers "*.Cu" "*.Mask") (remove_unused_layers no) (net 14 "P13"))
  (pad "29" thru_hole circle (at 0 -35.56 90) (size 1.7 1.7) (drill 1) (layers "*.Cu" "*.Mask") (remove_unused_layers no) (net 11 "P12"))
  (pad "30" thru_hole circle (at -2.54 -35.56 90) (size 1.7 1.7) (drill 1) (layers "*.Cu" "*.Mask") (remove_unused_layers no) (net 12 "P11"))
  (pad "31" thru_hole circle (at 0 -38.1 90) (size 1.7 1.7) (drill 1) (layers "*.Cu" "*.Mask") (remove_unused_layers no) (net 9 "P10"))
  (pad "32" thru_hole circle (at -2.54 -38.1 90) (size 1.7 1.7) (drill 1) (layers "*.Cu" "*.Mask") (remove_unused_layers no) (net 10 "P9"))
  (pad "33" thru_hole circle (at 0 -40.64 90) (size 1.7 1.7) (drill 1) (layers "*.Cu" "*.Mask") (remove_unused_layers no) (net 7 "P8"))
  (pad "34" thru_hole circle (at -2.54 -40.64 90) (size 1.7 1.7) (drill 1) (layers "*.Cu" "*.Mask") (remove_unused_layers no) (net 8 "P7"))
  (pad "35" thru_hole circle (at 0 -43.18 90) (size 1.7 1.7) (drill 1) (layers "*.Cu" "*.Mask") (remove_unused_layers no) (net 5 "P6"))
  (pad "36" thru_hole circle (at -2.54 -43.18 90) (size 1.7 1.7) (drill 1) (layers "*.Cu" "*.Mask") (remove_unused_layers no) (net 6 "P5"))
  (pad "37" thru_hole circle (at 0 -45.72 90) (size 1.7 1.7) (drill 1) (layers "*.Cu" "*.Mask") (remove_unused_layers no) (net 3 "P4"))
  (pad "38" thru_hole circle (at -2.54 -45.72 90) (size 1.7 1.7) (drill 1) (layers "*.Cu" "*.Mask") (remove_unused_layers no) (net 4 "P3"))
  (pad "39" thru_hole circle (at 0 -48.26 90) (size 1.7 1.7) (drill 1) (layers "*.Cu" "*.Mask") (remove_unused_layers no) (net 1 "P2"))
  (pad "40" thru_hole circle (at -2.54 -48.26 90) (size 1.7 1.7) (drill 1) (layers "*.Cu" "*.Mask") (remove_unused_layers no) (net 2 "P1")))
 (gr_line (start 100 60) (end 165 60) (stroke (width 0.1) (type default)) (layer "Edge.Cuts"))
 (gr_line (start 165 74) (end 100 74) (stroke (width 0.1) (type default)) (layer "Edge.Cuts"))
 (gr_line (start 165 60) (end 165 74) (stroke (width 0.1) (type default)) (layer "Edge.Cuts"))
 (gr_line (start 100 74) (end 100 60) (stroke (width 0.1) (type default)) (layer "Edge.Cuts"))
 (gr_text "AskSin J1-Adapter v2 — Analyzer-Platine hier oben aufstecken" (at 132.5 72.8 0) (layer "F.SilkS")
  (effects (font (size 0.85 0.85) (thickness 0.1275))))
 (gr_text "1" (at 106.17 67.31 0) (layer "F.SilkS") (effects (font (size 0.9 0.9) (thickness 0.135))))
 (segment (start 108.37 64.769999) (end 108.37 67.31) (width 0.5) (layer "F.Cu") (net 2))
 (segment (start 108.37 62.23) (end 109.64 63.5) (width 0.35) (layer "B.Cu") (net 1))
 (segment (start 109.64 63.5) (end 109.64 68.58) (width 0.35) (layer "B.Cu") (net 1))
 (segment (start 109.64 68.58) (end 108.37 69.85) (width 0.35) (layer "B.Cu") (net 1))
 (segment (start 110.91 64.769999) (end 110.91 67.31) (width 0.35) (layer "F.Cu") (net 4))
 (segment (start 110.91 62.23) (end 112.18 63.5) (width 0.35) (layer "B.Cu") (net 3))
 (segment (start 112.18 63.5) (end 112.18 68.58) (width 0.35) (layer "B.Cu") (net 3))
 (segment (start 112.18 68.58) (end 110.91 69.85) (width 0.35) (layer "B.Cu") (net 3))
 (segment (start 113.45 64.769999) (end 113.45 67.31) (width 0.35) (layer "F.Cu") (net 6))
 (segment (start 114.72 68.58) (end 113.45 69.85) (width 0.35) (layer "B.Cu") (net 5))
 (segment (start 113.45 62.23) (end 114.72 63.5) (width 0.35) (layer "B.Cu") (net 5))
 (segment (start 114.72 63.5) (end 114.72 68.58) (width 0.35) (layer "B.Cu") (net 5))
 (segment (start 115.99 64.769999) (end 115.99 67.31) (width 0.35) (layer "F.Cu") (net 8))
 (segment (start 115.99 62.23) (end 117.26 63.5) (width 0.35) (layer "B.Cu") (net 7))
 (segment (start 117.26 68.58) (end 115.99 69.85) (width 0.35) (layer "B.Cu") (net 7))
 (segment (start 117.26 63.5) (end 117.26 68.58) (width 0.35) (layer "B.Cu") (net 7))
 (segment (start 118.53 64.769999) (end 118.53 67.31) (width 0.5) (layer "F.Cu") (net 10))
 (segment (start 118.53 62.23) (end 119.8 63.5) (width 0.35) (layer "B.Cu") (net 9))
 (segment (start 119.8 63.5) (end 119.8 68.58) (width 0.35) (layer "B.Cu") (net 9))
 (segment (start 119.8 68.58) (end 118.53 69.85) (width 0.35) (layer "B.Cu") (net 9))
 (segment (start 121.07 64.769999) (end 121.07 67.31) (width 0.35) (layer "F.Cu") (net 12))
 (segment (start 122.34 63.5) (end 122.34 68.58) (width 0.35) (layer "B.Cu") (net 11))
 (segment (start 121.07 62.23) (end 122.34 63.5) (width 0.35) (layer "B.Cu") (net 11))
 (segment (start 122.34 68.58) (end 121.07 69.85) (width 0.35) (layer "B.Cu") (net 11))
 (segment (start 123.61 64.769999) (end 123.61 67.31) (width 0.35) (layer "F.Cu") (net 14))
 (segment (start 124.88 68.58) (end 123.61 69.85) (width 0.35) (layer "B.Cu") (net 13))
 (segment (start 124.88 63.5) (end 124.88 68.58) (width 0.35) (layer "B.Cu") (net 13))
 (segment (start 123.61 62.23) (end 124.88 63.5) (width 0.35) (layer "B.Cu") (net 13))
 (segment (start 126.15 64.769999) (end 126.15 67.31) (width 0.35) (layer "F.Cu") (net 16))
 (segment (start 127.42 68.58) (end 126.15 69.85) (width 0.35) (layer "B.Cu") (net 15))
 (segment (start 126.15 62.23) (end 127.42 63.5) (width 0.35) (layer "B.Cu") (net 15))
 (segment (start 127.42 63.5) (end 127.42 68.58) (width 0.35) (layer "B.Cu") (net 15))
 (segment (start 128.69 64.769999) (end 128.69 67.31) (width 0.5) (layer "F.Cu") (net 18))
 (segment (start 129.96 68.58) (end 128.69 69.85) (width 0.35) (layer "B.Cu") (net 17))
 (segment (start 128.69 62.23) (end 129.96 63.5) (width 0.35) (layer "B.Cu") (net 17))
 (segment (start 129.96 63.5) (end 129.96 68.58) (width 0.35) (layer "B.Cu") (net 17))
 (segment (start 131.229999 64.769999) (end 131.229999 67.31) (width 0.35) (layer "F.Cu") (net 20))
 (segment (start 132.5 63.5) (end 132.5 68.58) (width 0.35) (layer "B.Cu") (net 19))
 (segment (start 131.229999 62.23) (end 132.5 63.5) (width 0.35) (layer "B.Cu") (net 19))
 (segment (start 132.5 68.58) (end 131.229999 69.85) (width 0.35) (layer "B.Cu") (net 19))
 (segment (start 133.77 64.769999) (end 133.77 67.31) (width 0.35) (layer "F.Cu") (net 22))
 (segment (start 133.77 62.23) (end 135.04 63.5) (width 0.35) (layer "B.Cu") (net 21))
 (segment (start 135.04 68.58) (end 133.77 69.85) (width 0.35) (layer "B.Cu") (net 21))
 (segment (start 135.04 63.5) (end 135.04 68.58) (width 0.35) (layer "B.Cu") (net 21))
 (segment (start 136.31 64.769999) (end 136.31 67.31) (width 0.35) (layer "F.Cu") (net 24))
 (segment (start 136.31 62.23) (end 137.58 63.5) (width 0.35) (layer "B.Cu") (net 23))
 (segment (start 137.58 63.5) (end 137.58 68.58) (width 0.35) (layer "B.Cu") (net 23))
 (segment (start 137.58 68.58) (end 136.31 69.85) (width 0.35) (layer "B.Cu") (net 23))
 (segment (start 138.85 64.769999) (end 138.85 67.31) (width 0.5) (layer "F.Cu") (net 26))
 (segment (start 140.12 63.5) (end 140.12 68.58) (width 0.35) (layer "B.Cu") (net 25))
 (segment (start 138.85 62.23) (end 140.12 63.5) (width 0.35) (layer "B.Cu") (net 25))
 (segment (start 140.12 68.58) (end 138.85 69.85) (width 0.35) (layer "B.Cu") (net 25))
 (segment (start 141.39 64.769999) (end 141.39 67.31) (width 0.35) (layer "F.Cu") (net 28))
 (segment (start 142.66 68.58) (end 141.39 69.85) (width 0.35) (layer "B.Cu") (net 27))
 (segment (start 141.39 62.23) (end 142.66 63.5) (width 0.35) (layer "B.Cu") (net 27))
 (segment (start 142.66 63.5) (end 142.66 68.58) (width 0.35) (layer "B.Cu") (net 27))
 (segment (start 143.93 64.769999) (end 143.93 67.31) (width 0.35) (layer "F.Cu") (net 30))
 (segment (start 143.93 62.23) (end 145.2 63.5) (width 0.35) (layer "B.Cu") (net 29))
 (segment (start 145.2 63.5) (end 145.2 68.58) (width 0.35) (layer "B.Cu") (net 29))
 (segment (start 145.2 68.58) (end 143.93 69.85) (width 0.35) (layer "B.Cu") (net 29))
 (segment (start 146.47 64.769999) (end 146.47 67.31) (width 0.35) (layer "F.Cu") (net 32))
 (segment (start 147.74 63.5) (end 147.74 68.58) (width 0.35) (layer "B.Cu") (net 31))
 (segment (start 146.47 62.23) (end 147.74 63.5) (width 0.35) (layer "B.Cu") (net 31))
 (segment (start 147.74 68.58) (end 146.47 69.85) (width 0.35) (layer "B.Cu") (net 31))
 (segment (start 149.01 64.769999) (end 149.01 67.31) (width 0.35) (layer "F.Cu") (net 34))
 (segment (start 149.01 62.23) (end 150.28 63.5) (width 0.35) (layer "B.Cu") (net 33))
 (segment (start 150.28 63.5) (end 150.28 68.58) (width 0.35) (layer "B.Cu") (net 33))
 (segment (start 150.28 68.58) (end 149.01 69.85) (width 0.35) (layer "B.Cu") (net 33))
 (segment (start 151.55 64.769999) (end 151.55 67.31) (width 0.35) (layer "F.Cu") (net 36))
 (segment (start 152.82 68.58) (end 151.55 69.85) (width 0.35) (layer "B.Cu") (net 35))
 (segment (start 151.55 62.23) (end 152.82 63.5) (width 0.35) (layer "B.Cu") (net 35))
 (segment (start 152.82 63.5) (end 152.82 68.58) (width 0.35) (layer "B.Cu") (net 35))
 (segment (start 154.09 64.769999) (end 154.09 67.31) (width 0.35) (layer "F.Cu") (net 38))
 (segment (start 155.36 68.58) (end 154.09 69.85) (width 0.35) (layer "B.Cu") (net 37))
 (segment (start 155.36 63.5) (end 155.36 68.58) (width 0.35) (layer "B.Cu") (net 37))
 (segment (start 154.09 62.23) (end 155.36 63.5) (width 0.35) (layer "B.Cu") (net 37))
 (segment (start 156.63 64.769999) (end 156.63 67.31) (width 0.5) (layer "F.Cu") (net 40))
 (segment (start 157.9 68.58) (end 156.63 69.85) (width 0.35) (layer "B.Cu") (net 39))
 (segment (start 156.63 62.23) (end 157.9 63.5) (width 0.35) (layer "B.Cu") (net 39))
 (segment (start 157.9 63.5) (end 157.9 68.58) (width 0.35) (layer "B.Cu") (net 39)))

